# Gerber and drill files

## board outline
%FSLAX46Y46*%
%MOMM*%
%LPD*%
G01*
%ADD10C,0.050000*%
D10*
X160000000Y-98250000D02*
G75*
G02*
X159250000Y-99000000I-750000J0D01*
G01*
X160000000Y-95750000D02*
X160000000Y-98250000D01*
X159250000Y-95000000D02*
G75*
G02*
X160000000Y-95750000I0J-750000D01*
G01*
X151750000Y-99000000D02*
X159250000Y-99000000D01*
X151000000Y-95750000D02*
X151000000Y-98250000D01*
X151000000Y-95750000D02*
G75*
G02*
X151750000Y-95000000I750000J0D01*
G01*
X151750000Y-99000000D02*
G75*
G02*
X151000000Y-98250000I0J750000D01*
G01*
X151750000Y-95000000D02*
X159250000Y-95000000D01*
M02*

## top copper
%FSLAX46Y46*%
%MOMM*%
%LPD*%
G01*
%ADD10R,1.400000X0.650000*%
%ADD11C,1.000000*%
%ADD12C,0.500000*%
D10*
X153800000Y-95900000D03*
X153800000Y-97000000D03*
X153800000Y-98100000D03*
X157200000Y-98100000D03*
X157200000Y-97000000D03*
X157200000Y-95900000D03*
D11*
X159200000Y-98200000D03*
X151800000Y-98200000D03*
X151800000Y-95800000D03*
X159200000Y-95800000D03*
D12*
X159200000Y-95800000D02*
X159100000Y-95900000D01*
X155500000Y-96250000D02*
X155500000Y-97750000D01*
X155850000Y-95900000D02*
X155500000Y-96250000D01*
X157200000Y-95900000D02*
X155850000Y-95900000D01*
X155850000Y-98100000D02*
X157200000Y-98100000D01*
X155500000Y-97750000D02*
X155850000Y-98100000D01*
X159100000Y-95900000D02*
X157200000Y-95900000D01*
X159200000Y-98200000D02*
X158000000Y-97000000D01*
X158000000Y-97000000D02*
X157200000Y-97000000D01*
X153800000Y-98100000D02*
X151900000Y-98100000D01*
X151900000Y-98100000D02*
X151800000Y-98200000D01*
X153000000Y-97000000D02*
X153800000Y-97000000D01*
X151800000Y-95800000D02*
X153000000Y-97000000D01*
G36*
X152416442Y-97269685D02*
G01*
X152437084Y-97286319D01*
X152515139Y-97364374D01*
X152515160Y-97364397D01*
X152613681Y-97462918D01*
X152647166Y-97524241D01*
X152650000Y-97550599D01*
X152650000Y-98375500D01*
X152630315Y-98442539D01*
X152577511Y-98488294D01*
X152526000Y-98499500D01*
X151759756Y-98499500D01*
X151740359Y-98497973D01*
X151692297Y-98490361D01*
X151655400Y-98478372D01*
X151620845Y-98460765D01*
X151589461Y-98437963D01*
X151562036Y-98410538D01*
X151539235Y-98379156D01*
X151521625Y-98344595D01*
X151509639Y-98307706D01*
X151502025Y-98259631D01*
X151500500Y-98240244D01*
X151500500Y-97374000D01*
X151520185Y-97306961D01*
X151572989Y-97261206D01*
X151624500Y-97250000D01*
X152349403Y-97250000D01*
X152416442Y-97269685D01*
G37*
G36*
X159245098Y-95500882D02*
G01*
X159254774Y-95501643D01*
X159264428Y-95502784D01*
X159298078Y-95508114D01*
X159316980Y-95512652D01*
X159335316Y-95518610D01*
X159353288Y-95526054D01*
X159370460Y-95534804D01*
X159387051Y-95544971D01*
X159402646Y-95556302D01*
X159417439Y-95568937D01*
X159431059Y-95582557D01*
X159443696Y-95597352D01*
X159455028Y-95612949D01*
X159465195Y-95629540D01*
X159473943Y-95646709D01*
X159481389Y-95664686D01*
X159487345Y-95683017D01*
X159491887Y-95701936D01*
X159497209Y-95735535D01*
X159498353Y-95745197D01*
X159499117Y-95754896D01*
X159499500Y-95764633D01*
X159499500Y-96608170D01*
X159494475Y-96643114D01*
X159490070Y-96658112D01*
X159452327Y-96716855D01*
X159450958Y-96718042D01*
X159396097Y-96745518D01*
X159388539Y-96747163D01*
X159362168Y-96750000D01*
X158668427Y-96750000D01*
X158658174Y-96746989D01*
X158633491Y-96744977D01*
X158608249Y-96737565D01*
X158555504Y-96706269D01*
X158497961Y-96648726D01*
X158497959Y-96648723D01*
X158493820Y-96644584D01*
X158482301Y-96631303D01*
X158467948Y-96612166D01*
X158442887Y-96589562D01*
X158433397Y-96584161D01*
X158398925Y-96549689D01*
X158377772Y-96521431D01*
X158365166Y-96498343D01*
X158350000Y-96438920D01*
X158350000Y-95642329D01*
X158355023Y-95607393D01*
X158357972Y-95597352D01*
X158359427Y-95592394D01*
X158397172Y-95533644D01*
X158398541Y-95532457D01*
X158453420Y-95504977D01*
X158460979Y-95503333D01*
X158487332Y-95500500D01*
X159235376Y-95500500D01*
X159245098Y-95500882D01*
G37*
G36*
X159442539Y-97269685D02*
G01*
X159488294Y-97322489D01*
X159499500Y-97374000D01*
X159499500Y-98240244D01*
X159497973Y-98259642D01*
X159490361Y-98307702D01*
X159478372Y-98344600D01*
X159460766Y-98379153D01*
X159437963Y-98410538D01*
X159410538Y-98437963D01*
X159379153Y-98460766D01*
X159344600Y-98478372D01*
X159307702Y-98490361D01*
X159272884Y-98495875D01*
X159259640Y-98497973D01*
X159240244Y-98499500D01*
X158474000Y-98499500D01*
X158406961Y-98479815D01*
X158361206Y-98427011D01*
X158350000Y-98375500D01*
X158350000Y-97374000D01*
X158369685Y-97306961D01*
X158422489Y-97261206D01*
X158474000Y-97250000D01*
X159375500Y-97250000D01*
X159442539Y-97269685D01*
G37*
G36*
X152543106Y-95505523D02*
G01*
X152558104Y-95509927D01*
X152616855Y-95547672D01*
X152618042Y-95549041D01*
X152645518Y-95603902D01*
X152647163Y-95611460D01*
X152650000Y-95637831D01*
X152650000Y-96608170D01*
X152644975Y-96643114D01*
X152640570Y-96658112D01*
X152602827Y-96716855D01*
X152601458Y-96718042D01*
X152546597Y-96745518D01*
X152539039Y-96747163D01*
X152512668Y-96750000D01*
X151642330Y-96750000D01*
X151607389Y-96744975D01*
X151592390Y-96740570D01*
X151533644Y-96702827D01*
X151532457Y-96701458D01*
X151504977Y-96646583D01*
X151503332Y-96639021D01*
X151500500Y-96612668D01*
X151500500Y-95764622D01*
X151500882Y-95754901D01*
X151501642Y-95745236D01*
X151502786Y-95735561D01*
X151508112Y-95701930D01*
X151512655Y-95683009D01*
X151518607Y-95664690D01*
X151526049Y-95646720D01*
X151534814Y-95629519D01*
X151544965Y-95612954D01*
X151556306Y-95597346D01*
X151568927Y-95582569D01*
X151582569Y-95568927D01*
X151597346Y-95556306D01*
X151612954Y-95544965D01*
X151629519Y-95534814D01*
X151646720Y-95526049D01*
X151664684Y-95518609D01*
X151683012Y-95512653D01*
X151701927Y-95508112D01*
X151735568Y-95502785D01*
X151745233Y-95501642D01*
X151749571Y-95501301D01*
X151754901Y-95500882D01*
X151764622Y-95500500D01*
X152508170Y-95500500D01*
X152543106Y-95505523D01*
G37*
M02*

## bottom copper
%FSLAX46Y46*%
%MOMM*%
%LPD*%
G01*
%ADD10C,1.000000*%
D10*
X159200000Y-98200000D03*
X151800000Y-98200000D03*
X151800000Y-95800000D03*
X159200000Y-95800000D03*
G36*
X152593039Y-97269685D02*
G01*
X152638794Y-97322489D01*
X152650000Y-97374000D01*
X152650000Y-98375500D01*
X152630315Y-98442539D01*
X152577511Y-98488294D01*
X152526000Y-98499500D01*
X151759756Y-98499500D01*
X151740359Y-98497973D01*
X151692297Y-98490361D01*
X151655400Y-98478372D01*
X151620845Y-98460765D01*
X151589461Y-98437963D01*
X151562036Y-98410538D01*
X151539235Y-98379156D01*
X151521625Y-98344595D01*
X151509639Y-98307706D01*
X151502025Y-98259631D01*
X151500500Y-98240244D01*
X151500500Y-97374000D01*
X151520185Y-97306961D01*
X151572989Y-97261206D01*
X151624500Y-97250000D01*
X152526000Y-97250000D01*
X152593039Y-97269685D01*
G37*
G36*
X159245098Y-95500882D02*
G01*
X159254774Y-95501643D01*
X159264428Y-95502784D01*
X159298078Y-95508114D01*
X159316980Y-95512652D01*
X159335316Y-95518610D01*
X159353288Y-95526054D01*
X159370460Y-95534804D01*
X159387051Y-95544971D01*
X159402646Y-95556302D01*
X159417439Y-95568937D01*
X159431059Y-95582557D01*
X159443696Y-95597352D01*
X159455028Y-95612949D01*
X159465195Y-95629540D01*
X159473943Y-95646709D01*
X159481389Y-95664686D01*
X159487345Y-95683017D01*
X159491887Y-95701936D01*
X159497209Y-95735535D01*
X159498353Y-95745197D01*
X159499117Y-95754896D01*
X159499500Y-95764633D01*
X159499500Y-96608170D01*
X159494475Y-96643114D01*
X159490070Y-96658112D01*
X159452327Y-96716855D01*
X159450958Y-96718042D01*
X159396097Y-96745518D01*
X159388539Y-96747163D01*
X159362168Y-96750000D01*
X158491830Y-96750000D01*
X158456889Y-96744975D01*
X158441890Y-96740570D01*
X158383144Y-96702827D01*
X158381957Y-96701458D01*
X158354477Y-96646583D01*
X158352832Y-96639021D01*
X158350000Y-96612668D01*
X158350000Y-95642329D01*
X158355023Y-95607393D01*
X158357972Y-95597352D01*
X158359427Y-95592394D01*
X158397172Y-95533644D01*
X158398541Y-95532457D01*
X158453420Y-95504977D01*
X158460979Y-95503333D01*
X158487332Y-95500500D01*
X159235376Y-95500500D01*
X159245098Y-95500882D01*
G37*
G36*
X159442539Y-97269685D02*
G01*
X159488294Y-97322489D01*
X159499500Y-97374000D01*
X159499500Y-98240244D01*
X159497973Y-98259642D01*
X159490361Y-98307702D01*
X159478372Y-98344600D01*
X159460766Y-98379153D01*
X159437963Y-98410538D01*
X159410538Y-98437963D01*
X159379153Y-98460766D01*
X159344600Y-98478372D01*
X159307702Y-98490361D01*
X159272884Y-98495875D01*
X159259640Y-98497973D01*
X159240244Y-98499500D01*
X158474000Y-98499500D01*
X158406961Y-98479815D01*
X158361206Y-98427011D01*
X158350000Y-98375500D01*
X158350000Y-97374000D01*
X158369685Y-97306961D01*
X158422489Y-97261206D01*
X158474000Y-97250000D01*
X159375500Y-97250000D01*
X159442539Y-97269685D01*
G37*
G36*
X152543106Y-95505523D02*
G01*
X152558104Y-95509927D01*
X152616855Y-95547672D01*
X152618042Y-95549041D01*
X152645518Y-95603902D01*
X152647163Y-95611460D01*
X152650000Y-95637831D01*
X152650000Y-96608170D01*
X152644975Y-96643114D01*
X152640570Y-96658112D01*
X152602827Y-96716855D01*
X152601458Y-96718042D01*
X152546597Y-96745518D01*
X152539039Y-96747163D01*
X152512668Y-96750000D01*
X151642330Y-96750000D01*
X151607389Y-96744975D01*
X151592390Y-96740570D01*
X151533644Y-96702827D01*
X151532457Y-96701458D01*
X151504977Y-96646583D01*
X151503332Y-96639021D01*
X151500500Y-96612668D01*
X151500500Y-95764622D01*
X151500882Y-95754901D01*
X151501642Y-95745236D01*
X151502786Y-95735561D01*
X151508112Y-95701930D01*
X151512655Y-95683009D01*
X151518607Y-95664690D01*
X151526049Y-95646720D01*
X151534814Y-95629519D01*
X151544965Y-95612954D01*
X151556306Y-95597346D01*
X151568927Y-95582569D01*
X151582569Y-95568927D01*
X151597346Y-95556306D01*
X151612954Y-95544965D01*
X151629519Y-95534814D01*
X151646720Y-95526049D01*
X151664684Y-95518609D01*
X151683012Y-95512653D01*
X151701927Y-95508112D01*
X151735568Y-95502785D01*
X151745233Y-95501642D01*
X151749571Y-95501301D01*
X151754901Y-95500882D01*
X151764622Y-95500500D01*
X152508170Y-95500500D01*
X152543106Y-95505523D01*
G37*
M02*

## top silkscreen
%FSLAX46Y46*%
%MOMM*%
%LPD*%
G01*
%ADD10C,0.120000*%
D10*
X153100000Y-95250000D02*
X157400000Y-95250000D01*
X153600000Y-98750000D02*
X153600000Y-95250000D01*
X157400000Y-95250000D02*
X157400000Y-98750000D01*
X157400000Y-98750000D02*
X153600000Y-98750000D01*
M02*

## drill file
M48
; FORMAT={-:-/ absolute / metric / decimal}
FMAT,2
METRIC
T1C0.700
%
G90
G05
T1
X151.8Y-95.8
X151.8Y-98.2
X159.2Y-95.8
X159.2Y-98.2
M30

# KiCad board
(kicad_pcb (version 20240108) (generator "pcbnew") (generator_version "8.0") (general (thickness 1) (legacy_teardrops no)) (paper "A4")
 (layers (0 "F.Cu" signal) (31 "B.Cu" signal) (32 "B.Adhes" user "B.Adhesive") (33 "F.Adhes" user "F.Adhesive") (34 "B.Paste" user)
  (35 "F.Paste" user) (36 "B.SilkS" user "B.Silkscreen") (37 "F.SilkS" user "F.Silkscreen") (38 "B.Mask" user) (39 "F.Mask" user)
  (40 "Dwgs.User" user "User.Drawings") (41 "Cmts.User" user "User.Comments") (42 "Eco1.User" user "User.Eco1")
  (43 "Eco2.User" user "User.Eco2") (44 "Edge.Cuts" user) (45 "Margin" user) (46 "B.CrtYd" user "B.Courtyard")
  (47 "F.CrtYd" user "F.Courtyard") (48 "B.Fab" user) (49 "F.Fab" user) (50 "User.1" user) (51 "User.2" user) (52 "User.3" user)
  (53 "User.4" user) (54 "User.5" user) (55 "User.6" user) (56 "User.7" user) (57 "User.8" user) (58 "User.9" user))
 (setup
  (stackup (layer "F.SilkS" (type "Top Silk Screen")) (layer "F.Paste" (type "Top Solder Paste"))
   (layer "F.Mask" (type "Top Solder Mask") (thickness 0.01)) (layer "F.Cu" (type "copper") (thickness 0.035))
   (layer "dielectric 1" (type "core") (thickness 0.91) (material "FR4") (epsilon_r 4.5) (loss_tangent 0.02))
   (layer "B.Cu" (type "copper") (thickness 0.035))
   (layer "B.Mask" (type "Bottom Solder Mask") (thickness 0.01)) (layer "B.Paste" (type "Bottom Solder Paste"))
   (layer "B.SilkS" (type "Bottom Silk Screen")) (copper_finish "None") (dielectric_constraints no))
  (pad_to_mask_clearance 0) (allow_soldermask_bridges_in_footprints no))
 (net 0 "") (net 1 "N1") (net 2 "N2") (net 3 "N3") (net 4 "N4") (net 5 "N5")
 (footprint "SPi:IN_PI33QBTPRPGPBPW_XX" (layer "F.Cu") (at 155.5 97 -90)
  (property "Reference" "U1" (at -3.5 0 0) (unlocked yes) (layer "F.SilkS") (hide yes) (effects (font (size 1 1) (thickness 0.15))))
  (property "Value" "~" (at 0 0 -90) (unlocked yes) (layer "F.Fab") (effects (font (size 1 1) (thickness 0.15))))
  (fp_line (start -1.75 2.4) (end -1.75 -1.9) (stroke (width 0.12) (type default)) (layer "F.SilkS"))
  (fp_line (start 1.75 1.9) (end -1.75 1.9) (stroke (width 0.12) (type default)) (layer "F.SilkS"))
  (fp_line (start -1.75 -1.9) (end 1.75 -1.9) (stroke (width 0.12) (type default)) (layer "F.SilkS"))
  (fp_line (start 1.75 -1.9) (end 1.75 1.9) (stroke (width 0.12) (type default)) (layer "F.SilkS"))
  (pad "1" smd rect (at -1.1 1.7 270) (size 0.65 1.4) (layers "F.Cu" "F.Paste" "F.Mask") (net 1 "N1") (thermal_bridge_angle 45))
  (pad "2" smd rect (at 0 1.7 270) (size 0.65 1.4) (layers "F.Cu" "F.Paste" "F.Mask") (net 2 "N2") (thermal_bridge_angle 45))
  (pad "3" smd rect (at 1.1 1.7 270) (size 0.65 1.4) (layers "F.Cu" "F.Paste" "F.Mask") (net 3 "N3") (thermal_bridge_angle 45))
  (pad "4" smd rect (at 1.1 -1.7 270) (size 0.65 1.4) (layers "F.Cu" "F.Paste" "F.Mask") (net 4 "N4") (thermal_bridge_angle 45))
  (pad "5" smd rect (at 0 -1.7 270) (size 0.65 1.4) (layers "F.Cu" "F.Paste" "F.Mask") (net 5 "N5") (thermal_bridge_angle 45))
  (pad "6" smd rect (at -1.1 -1.7 270) (size 0.65 1.4) (layers "F.Cu" "F.Paste" "F.Mask") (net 4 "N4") (thermal_bridge_angle 45)))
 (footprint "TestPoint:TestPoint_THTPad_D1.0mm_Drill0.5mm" (layer "F.Cu") (at 159.2 98.2)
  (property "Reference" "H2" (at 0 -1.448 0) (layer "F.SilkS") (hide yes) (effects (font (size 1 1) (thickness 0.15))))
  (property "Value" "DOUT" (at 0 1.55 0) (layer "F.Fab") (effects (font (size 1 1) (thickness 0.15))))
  (pad "1" thru_hole circle (at 0 0) (size 1 1) (drill 0.7) (layers "*.Cu" "*.Mask") (remove_unused_layers no) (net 5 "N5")))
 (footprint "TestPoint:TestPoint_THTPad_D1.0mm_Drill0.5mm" (layer "F.Cu") (at 151.8 98.2)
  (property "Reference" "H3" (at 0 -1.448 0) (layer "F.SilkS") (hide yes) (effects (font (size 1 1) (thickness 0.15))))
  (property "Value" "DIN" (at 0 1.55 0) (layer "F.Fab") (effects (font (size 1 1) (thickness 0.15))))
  (pad "1" thru_hole circle (at 0 0) (size 1 1) (drill 0.7) (layers "*.Cu" "*.Mask") (remove_unused_layers no) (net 3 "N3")))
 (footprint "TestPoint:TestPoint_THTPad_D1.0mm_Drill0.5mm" (layer "F.Cu") (at 151.8 95.8)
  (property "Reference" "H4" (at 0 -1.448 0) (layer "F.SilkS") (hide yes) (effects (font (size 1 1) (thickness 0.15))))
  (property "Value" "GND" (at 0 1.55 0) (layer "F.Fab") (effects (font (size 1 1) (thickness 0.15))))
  (pad "1" thru_hole circle (at 0 0) (size 1 1) (drill 0.7) (layers "*.Cu" "*.Mask") (remove_unused_layers no) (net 2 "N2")))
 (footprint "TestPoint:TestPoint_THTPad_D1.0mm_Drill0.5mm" (layer "F.Cu") (at 159.2 95.8)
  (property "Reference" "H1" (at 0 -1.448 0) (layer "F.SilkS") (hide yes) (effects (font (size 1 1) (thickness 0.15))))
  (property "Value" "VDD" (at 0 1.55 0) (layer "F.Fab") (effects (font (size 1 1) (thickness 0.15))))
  (pad "1" thru_hole circle (at 0 0) (size 1 1) (drill 0.7) (layers "*.Cu" "*.Mask") (remove_unused_layers no) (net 4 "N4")))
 (gr_arc (start 160 98.25) (mid 159.78033 98.78033) (end 159.25 99) (stroke (width 0.05) (type default)) (layer "Edge.Cuts"))
 (gr_line (start 160 95.75) (end 160 98.25) (stroke (width 0.05) (type default)) (layer "Edge.Cuts"))
 (gr_arc (start 159.25 95) (mid 159.78033 95.21967) (end 160 95.75) (stroke (width 0.05) (type default)) (layer "Edge.Cuts"))
 (gr_line (start 151.75 99) (end 159.25 99) (stroke (width 0.05) (type default)) (layer "Edge.Cuts"))
 (gr_line (start 151 95.75) (end 151 98.25) (stroke (width 0.05) (type default)) (layer "Edge.Cuts"))
 (gr_arc (start 151 95.75) (mid 151.21967 95.21967) (end 151.75 95) (stroke (width 0.05) (type default)) (layer "Edge.Cuts"))
 (gr_arc (start 151.75 99) (mid 151.21967 98.78033) (end 151 98.25) (stroke (width 0.05) (type default)) (layer "Edge.Cuts"))
 (gr_line (start 151.75 95) (end 159.25 95) (stroke (width 0.05) (type default)) (layer "Edge.Cuts"))
 (segment (start 159.2 95.8) (end 159.1 95.9) (width 0.5) (layer "F.Cu") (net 4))
 (segment (start 155.5 96.25) (end 155.5 97.75) (width 0.5) (layer "F.Cu") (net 4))
 (segment (start 155.85 95.9) (end 155.5 96.25) (width 0.5) (layer "F.Cu") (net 4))
 (segment (start 157.2 95.9) (end 155.85 95.9) (width 0.5) (layer "F.Cu") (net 4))
 (segment (start 155.85 98.1) (end 157.2 98.1) (width 0.5) (layer "F.Cu") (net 4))
 (segment (start 155.5 97.75) (end 155.85 98.1) (width 0.5) (layer "F.Cu") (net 4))
 (segment (start 159.1 95.9) (end 157.2 95.9) (width 0.5) (layer "F.Cu") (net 4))
 (segment (start 159.2 98.2) (end 158 97) (width 0.5) (layer "F.Cu") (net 5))
 (segment (start 158 97) (end 157.2 97) (width 0.5) (layer "F.Cu") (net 5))
 (segment (start 153.8 98.1) (end 151.9 98.1) (width 0.5) (layer "F.Cu") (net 3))
 (segment (start 151.9 98.1) (end 151.8 98.2) (width 0.5) (layer "F.Cu") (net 3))
 (segment (start 153 97) (end 153.8 97) (width 0.5) (layer "F.Cu") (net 2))
 (segment (start 151.8 95.8) (end 153 97) (width 0.5) (layer "F.Cu") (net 2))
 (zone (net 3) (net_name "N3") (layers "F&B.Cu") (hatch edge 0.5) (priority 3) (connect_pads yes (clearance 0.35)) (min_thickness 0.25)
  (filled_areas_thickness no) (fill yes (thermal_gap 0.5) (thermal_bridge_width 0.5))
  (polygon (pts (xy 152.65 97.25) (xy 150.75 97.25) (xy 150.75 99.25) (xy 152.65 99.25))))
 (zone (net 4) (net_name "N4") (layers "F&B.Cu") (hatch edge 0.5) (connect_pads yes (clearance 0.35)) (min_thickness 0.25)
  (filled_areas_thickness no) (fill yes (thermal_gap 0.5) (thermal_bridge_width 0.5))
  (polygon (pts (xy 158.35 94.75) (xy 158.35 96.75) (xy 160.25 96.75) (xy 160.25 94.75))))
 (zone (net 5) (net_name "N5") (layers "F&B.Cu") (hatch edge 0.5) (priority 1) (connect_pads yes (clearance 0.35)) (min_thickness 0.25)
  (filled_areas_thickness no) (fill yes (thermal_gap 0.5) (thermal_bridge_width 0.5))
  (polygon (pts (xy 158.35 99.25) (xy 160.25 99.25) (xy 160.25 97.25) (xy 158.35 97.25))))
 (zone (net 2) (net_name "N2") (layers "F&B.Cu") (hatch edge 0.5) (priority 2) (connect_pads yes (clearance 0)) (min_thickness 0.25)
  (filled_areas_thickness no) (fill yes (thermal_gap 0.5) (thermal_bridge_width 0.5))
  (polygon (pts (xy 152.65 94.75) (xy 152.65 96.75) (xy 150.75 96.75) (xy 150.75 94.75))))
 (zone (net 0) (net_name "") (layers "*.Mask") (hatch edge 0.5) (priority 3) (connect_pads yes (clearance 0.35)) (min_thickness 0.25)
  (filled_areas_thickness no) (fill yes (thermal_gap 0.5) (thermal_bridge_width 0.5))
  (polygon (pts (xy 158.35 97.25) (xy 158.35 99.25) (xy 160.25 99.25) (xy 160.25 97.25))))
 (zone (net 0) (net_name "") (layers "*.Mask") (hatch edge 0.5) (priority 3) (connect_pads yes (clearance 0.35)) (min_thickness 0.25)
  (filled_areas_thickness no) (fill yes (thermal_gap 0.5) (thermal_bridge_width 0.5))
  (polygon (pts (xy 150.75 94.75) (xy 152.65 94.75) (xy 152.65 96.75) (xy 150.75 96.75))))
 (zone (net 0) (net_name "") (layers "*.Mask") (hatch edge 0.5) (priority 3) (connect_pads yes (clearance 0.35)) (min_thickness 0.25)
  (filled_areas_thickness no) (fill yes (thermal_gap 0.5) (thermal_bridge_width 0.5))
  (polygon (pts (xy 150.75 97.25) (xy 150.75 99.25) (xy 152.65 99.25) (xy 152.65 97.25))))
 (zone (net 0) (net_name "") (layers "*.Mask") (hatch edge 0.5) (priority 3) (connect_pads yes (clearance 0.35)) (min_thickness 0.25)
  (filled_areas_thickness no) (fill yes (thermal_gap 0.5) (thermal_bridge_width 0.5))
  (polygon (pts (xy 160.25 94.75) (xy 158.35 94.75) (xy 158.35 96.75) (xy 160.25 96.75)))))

